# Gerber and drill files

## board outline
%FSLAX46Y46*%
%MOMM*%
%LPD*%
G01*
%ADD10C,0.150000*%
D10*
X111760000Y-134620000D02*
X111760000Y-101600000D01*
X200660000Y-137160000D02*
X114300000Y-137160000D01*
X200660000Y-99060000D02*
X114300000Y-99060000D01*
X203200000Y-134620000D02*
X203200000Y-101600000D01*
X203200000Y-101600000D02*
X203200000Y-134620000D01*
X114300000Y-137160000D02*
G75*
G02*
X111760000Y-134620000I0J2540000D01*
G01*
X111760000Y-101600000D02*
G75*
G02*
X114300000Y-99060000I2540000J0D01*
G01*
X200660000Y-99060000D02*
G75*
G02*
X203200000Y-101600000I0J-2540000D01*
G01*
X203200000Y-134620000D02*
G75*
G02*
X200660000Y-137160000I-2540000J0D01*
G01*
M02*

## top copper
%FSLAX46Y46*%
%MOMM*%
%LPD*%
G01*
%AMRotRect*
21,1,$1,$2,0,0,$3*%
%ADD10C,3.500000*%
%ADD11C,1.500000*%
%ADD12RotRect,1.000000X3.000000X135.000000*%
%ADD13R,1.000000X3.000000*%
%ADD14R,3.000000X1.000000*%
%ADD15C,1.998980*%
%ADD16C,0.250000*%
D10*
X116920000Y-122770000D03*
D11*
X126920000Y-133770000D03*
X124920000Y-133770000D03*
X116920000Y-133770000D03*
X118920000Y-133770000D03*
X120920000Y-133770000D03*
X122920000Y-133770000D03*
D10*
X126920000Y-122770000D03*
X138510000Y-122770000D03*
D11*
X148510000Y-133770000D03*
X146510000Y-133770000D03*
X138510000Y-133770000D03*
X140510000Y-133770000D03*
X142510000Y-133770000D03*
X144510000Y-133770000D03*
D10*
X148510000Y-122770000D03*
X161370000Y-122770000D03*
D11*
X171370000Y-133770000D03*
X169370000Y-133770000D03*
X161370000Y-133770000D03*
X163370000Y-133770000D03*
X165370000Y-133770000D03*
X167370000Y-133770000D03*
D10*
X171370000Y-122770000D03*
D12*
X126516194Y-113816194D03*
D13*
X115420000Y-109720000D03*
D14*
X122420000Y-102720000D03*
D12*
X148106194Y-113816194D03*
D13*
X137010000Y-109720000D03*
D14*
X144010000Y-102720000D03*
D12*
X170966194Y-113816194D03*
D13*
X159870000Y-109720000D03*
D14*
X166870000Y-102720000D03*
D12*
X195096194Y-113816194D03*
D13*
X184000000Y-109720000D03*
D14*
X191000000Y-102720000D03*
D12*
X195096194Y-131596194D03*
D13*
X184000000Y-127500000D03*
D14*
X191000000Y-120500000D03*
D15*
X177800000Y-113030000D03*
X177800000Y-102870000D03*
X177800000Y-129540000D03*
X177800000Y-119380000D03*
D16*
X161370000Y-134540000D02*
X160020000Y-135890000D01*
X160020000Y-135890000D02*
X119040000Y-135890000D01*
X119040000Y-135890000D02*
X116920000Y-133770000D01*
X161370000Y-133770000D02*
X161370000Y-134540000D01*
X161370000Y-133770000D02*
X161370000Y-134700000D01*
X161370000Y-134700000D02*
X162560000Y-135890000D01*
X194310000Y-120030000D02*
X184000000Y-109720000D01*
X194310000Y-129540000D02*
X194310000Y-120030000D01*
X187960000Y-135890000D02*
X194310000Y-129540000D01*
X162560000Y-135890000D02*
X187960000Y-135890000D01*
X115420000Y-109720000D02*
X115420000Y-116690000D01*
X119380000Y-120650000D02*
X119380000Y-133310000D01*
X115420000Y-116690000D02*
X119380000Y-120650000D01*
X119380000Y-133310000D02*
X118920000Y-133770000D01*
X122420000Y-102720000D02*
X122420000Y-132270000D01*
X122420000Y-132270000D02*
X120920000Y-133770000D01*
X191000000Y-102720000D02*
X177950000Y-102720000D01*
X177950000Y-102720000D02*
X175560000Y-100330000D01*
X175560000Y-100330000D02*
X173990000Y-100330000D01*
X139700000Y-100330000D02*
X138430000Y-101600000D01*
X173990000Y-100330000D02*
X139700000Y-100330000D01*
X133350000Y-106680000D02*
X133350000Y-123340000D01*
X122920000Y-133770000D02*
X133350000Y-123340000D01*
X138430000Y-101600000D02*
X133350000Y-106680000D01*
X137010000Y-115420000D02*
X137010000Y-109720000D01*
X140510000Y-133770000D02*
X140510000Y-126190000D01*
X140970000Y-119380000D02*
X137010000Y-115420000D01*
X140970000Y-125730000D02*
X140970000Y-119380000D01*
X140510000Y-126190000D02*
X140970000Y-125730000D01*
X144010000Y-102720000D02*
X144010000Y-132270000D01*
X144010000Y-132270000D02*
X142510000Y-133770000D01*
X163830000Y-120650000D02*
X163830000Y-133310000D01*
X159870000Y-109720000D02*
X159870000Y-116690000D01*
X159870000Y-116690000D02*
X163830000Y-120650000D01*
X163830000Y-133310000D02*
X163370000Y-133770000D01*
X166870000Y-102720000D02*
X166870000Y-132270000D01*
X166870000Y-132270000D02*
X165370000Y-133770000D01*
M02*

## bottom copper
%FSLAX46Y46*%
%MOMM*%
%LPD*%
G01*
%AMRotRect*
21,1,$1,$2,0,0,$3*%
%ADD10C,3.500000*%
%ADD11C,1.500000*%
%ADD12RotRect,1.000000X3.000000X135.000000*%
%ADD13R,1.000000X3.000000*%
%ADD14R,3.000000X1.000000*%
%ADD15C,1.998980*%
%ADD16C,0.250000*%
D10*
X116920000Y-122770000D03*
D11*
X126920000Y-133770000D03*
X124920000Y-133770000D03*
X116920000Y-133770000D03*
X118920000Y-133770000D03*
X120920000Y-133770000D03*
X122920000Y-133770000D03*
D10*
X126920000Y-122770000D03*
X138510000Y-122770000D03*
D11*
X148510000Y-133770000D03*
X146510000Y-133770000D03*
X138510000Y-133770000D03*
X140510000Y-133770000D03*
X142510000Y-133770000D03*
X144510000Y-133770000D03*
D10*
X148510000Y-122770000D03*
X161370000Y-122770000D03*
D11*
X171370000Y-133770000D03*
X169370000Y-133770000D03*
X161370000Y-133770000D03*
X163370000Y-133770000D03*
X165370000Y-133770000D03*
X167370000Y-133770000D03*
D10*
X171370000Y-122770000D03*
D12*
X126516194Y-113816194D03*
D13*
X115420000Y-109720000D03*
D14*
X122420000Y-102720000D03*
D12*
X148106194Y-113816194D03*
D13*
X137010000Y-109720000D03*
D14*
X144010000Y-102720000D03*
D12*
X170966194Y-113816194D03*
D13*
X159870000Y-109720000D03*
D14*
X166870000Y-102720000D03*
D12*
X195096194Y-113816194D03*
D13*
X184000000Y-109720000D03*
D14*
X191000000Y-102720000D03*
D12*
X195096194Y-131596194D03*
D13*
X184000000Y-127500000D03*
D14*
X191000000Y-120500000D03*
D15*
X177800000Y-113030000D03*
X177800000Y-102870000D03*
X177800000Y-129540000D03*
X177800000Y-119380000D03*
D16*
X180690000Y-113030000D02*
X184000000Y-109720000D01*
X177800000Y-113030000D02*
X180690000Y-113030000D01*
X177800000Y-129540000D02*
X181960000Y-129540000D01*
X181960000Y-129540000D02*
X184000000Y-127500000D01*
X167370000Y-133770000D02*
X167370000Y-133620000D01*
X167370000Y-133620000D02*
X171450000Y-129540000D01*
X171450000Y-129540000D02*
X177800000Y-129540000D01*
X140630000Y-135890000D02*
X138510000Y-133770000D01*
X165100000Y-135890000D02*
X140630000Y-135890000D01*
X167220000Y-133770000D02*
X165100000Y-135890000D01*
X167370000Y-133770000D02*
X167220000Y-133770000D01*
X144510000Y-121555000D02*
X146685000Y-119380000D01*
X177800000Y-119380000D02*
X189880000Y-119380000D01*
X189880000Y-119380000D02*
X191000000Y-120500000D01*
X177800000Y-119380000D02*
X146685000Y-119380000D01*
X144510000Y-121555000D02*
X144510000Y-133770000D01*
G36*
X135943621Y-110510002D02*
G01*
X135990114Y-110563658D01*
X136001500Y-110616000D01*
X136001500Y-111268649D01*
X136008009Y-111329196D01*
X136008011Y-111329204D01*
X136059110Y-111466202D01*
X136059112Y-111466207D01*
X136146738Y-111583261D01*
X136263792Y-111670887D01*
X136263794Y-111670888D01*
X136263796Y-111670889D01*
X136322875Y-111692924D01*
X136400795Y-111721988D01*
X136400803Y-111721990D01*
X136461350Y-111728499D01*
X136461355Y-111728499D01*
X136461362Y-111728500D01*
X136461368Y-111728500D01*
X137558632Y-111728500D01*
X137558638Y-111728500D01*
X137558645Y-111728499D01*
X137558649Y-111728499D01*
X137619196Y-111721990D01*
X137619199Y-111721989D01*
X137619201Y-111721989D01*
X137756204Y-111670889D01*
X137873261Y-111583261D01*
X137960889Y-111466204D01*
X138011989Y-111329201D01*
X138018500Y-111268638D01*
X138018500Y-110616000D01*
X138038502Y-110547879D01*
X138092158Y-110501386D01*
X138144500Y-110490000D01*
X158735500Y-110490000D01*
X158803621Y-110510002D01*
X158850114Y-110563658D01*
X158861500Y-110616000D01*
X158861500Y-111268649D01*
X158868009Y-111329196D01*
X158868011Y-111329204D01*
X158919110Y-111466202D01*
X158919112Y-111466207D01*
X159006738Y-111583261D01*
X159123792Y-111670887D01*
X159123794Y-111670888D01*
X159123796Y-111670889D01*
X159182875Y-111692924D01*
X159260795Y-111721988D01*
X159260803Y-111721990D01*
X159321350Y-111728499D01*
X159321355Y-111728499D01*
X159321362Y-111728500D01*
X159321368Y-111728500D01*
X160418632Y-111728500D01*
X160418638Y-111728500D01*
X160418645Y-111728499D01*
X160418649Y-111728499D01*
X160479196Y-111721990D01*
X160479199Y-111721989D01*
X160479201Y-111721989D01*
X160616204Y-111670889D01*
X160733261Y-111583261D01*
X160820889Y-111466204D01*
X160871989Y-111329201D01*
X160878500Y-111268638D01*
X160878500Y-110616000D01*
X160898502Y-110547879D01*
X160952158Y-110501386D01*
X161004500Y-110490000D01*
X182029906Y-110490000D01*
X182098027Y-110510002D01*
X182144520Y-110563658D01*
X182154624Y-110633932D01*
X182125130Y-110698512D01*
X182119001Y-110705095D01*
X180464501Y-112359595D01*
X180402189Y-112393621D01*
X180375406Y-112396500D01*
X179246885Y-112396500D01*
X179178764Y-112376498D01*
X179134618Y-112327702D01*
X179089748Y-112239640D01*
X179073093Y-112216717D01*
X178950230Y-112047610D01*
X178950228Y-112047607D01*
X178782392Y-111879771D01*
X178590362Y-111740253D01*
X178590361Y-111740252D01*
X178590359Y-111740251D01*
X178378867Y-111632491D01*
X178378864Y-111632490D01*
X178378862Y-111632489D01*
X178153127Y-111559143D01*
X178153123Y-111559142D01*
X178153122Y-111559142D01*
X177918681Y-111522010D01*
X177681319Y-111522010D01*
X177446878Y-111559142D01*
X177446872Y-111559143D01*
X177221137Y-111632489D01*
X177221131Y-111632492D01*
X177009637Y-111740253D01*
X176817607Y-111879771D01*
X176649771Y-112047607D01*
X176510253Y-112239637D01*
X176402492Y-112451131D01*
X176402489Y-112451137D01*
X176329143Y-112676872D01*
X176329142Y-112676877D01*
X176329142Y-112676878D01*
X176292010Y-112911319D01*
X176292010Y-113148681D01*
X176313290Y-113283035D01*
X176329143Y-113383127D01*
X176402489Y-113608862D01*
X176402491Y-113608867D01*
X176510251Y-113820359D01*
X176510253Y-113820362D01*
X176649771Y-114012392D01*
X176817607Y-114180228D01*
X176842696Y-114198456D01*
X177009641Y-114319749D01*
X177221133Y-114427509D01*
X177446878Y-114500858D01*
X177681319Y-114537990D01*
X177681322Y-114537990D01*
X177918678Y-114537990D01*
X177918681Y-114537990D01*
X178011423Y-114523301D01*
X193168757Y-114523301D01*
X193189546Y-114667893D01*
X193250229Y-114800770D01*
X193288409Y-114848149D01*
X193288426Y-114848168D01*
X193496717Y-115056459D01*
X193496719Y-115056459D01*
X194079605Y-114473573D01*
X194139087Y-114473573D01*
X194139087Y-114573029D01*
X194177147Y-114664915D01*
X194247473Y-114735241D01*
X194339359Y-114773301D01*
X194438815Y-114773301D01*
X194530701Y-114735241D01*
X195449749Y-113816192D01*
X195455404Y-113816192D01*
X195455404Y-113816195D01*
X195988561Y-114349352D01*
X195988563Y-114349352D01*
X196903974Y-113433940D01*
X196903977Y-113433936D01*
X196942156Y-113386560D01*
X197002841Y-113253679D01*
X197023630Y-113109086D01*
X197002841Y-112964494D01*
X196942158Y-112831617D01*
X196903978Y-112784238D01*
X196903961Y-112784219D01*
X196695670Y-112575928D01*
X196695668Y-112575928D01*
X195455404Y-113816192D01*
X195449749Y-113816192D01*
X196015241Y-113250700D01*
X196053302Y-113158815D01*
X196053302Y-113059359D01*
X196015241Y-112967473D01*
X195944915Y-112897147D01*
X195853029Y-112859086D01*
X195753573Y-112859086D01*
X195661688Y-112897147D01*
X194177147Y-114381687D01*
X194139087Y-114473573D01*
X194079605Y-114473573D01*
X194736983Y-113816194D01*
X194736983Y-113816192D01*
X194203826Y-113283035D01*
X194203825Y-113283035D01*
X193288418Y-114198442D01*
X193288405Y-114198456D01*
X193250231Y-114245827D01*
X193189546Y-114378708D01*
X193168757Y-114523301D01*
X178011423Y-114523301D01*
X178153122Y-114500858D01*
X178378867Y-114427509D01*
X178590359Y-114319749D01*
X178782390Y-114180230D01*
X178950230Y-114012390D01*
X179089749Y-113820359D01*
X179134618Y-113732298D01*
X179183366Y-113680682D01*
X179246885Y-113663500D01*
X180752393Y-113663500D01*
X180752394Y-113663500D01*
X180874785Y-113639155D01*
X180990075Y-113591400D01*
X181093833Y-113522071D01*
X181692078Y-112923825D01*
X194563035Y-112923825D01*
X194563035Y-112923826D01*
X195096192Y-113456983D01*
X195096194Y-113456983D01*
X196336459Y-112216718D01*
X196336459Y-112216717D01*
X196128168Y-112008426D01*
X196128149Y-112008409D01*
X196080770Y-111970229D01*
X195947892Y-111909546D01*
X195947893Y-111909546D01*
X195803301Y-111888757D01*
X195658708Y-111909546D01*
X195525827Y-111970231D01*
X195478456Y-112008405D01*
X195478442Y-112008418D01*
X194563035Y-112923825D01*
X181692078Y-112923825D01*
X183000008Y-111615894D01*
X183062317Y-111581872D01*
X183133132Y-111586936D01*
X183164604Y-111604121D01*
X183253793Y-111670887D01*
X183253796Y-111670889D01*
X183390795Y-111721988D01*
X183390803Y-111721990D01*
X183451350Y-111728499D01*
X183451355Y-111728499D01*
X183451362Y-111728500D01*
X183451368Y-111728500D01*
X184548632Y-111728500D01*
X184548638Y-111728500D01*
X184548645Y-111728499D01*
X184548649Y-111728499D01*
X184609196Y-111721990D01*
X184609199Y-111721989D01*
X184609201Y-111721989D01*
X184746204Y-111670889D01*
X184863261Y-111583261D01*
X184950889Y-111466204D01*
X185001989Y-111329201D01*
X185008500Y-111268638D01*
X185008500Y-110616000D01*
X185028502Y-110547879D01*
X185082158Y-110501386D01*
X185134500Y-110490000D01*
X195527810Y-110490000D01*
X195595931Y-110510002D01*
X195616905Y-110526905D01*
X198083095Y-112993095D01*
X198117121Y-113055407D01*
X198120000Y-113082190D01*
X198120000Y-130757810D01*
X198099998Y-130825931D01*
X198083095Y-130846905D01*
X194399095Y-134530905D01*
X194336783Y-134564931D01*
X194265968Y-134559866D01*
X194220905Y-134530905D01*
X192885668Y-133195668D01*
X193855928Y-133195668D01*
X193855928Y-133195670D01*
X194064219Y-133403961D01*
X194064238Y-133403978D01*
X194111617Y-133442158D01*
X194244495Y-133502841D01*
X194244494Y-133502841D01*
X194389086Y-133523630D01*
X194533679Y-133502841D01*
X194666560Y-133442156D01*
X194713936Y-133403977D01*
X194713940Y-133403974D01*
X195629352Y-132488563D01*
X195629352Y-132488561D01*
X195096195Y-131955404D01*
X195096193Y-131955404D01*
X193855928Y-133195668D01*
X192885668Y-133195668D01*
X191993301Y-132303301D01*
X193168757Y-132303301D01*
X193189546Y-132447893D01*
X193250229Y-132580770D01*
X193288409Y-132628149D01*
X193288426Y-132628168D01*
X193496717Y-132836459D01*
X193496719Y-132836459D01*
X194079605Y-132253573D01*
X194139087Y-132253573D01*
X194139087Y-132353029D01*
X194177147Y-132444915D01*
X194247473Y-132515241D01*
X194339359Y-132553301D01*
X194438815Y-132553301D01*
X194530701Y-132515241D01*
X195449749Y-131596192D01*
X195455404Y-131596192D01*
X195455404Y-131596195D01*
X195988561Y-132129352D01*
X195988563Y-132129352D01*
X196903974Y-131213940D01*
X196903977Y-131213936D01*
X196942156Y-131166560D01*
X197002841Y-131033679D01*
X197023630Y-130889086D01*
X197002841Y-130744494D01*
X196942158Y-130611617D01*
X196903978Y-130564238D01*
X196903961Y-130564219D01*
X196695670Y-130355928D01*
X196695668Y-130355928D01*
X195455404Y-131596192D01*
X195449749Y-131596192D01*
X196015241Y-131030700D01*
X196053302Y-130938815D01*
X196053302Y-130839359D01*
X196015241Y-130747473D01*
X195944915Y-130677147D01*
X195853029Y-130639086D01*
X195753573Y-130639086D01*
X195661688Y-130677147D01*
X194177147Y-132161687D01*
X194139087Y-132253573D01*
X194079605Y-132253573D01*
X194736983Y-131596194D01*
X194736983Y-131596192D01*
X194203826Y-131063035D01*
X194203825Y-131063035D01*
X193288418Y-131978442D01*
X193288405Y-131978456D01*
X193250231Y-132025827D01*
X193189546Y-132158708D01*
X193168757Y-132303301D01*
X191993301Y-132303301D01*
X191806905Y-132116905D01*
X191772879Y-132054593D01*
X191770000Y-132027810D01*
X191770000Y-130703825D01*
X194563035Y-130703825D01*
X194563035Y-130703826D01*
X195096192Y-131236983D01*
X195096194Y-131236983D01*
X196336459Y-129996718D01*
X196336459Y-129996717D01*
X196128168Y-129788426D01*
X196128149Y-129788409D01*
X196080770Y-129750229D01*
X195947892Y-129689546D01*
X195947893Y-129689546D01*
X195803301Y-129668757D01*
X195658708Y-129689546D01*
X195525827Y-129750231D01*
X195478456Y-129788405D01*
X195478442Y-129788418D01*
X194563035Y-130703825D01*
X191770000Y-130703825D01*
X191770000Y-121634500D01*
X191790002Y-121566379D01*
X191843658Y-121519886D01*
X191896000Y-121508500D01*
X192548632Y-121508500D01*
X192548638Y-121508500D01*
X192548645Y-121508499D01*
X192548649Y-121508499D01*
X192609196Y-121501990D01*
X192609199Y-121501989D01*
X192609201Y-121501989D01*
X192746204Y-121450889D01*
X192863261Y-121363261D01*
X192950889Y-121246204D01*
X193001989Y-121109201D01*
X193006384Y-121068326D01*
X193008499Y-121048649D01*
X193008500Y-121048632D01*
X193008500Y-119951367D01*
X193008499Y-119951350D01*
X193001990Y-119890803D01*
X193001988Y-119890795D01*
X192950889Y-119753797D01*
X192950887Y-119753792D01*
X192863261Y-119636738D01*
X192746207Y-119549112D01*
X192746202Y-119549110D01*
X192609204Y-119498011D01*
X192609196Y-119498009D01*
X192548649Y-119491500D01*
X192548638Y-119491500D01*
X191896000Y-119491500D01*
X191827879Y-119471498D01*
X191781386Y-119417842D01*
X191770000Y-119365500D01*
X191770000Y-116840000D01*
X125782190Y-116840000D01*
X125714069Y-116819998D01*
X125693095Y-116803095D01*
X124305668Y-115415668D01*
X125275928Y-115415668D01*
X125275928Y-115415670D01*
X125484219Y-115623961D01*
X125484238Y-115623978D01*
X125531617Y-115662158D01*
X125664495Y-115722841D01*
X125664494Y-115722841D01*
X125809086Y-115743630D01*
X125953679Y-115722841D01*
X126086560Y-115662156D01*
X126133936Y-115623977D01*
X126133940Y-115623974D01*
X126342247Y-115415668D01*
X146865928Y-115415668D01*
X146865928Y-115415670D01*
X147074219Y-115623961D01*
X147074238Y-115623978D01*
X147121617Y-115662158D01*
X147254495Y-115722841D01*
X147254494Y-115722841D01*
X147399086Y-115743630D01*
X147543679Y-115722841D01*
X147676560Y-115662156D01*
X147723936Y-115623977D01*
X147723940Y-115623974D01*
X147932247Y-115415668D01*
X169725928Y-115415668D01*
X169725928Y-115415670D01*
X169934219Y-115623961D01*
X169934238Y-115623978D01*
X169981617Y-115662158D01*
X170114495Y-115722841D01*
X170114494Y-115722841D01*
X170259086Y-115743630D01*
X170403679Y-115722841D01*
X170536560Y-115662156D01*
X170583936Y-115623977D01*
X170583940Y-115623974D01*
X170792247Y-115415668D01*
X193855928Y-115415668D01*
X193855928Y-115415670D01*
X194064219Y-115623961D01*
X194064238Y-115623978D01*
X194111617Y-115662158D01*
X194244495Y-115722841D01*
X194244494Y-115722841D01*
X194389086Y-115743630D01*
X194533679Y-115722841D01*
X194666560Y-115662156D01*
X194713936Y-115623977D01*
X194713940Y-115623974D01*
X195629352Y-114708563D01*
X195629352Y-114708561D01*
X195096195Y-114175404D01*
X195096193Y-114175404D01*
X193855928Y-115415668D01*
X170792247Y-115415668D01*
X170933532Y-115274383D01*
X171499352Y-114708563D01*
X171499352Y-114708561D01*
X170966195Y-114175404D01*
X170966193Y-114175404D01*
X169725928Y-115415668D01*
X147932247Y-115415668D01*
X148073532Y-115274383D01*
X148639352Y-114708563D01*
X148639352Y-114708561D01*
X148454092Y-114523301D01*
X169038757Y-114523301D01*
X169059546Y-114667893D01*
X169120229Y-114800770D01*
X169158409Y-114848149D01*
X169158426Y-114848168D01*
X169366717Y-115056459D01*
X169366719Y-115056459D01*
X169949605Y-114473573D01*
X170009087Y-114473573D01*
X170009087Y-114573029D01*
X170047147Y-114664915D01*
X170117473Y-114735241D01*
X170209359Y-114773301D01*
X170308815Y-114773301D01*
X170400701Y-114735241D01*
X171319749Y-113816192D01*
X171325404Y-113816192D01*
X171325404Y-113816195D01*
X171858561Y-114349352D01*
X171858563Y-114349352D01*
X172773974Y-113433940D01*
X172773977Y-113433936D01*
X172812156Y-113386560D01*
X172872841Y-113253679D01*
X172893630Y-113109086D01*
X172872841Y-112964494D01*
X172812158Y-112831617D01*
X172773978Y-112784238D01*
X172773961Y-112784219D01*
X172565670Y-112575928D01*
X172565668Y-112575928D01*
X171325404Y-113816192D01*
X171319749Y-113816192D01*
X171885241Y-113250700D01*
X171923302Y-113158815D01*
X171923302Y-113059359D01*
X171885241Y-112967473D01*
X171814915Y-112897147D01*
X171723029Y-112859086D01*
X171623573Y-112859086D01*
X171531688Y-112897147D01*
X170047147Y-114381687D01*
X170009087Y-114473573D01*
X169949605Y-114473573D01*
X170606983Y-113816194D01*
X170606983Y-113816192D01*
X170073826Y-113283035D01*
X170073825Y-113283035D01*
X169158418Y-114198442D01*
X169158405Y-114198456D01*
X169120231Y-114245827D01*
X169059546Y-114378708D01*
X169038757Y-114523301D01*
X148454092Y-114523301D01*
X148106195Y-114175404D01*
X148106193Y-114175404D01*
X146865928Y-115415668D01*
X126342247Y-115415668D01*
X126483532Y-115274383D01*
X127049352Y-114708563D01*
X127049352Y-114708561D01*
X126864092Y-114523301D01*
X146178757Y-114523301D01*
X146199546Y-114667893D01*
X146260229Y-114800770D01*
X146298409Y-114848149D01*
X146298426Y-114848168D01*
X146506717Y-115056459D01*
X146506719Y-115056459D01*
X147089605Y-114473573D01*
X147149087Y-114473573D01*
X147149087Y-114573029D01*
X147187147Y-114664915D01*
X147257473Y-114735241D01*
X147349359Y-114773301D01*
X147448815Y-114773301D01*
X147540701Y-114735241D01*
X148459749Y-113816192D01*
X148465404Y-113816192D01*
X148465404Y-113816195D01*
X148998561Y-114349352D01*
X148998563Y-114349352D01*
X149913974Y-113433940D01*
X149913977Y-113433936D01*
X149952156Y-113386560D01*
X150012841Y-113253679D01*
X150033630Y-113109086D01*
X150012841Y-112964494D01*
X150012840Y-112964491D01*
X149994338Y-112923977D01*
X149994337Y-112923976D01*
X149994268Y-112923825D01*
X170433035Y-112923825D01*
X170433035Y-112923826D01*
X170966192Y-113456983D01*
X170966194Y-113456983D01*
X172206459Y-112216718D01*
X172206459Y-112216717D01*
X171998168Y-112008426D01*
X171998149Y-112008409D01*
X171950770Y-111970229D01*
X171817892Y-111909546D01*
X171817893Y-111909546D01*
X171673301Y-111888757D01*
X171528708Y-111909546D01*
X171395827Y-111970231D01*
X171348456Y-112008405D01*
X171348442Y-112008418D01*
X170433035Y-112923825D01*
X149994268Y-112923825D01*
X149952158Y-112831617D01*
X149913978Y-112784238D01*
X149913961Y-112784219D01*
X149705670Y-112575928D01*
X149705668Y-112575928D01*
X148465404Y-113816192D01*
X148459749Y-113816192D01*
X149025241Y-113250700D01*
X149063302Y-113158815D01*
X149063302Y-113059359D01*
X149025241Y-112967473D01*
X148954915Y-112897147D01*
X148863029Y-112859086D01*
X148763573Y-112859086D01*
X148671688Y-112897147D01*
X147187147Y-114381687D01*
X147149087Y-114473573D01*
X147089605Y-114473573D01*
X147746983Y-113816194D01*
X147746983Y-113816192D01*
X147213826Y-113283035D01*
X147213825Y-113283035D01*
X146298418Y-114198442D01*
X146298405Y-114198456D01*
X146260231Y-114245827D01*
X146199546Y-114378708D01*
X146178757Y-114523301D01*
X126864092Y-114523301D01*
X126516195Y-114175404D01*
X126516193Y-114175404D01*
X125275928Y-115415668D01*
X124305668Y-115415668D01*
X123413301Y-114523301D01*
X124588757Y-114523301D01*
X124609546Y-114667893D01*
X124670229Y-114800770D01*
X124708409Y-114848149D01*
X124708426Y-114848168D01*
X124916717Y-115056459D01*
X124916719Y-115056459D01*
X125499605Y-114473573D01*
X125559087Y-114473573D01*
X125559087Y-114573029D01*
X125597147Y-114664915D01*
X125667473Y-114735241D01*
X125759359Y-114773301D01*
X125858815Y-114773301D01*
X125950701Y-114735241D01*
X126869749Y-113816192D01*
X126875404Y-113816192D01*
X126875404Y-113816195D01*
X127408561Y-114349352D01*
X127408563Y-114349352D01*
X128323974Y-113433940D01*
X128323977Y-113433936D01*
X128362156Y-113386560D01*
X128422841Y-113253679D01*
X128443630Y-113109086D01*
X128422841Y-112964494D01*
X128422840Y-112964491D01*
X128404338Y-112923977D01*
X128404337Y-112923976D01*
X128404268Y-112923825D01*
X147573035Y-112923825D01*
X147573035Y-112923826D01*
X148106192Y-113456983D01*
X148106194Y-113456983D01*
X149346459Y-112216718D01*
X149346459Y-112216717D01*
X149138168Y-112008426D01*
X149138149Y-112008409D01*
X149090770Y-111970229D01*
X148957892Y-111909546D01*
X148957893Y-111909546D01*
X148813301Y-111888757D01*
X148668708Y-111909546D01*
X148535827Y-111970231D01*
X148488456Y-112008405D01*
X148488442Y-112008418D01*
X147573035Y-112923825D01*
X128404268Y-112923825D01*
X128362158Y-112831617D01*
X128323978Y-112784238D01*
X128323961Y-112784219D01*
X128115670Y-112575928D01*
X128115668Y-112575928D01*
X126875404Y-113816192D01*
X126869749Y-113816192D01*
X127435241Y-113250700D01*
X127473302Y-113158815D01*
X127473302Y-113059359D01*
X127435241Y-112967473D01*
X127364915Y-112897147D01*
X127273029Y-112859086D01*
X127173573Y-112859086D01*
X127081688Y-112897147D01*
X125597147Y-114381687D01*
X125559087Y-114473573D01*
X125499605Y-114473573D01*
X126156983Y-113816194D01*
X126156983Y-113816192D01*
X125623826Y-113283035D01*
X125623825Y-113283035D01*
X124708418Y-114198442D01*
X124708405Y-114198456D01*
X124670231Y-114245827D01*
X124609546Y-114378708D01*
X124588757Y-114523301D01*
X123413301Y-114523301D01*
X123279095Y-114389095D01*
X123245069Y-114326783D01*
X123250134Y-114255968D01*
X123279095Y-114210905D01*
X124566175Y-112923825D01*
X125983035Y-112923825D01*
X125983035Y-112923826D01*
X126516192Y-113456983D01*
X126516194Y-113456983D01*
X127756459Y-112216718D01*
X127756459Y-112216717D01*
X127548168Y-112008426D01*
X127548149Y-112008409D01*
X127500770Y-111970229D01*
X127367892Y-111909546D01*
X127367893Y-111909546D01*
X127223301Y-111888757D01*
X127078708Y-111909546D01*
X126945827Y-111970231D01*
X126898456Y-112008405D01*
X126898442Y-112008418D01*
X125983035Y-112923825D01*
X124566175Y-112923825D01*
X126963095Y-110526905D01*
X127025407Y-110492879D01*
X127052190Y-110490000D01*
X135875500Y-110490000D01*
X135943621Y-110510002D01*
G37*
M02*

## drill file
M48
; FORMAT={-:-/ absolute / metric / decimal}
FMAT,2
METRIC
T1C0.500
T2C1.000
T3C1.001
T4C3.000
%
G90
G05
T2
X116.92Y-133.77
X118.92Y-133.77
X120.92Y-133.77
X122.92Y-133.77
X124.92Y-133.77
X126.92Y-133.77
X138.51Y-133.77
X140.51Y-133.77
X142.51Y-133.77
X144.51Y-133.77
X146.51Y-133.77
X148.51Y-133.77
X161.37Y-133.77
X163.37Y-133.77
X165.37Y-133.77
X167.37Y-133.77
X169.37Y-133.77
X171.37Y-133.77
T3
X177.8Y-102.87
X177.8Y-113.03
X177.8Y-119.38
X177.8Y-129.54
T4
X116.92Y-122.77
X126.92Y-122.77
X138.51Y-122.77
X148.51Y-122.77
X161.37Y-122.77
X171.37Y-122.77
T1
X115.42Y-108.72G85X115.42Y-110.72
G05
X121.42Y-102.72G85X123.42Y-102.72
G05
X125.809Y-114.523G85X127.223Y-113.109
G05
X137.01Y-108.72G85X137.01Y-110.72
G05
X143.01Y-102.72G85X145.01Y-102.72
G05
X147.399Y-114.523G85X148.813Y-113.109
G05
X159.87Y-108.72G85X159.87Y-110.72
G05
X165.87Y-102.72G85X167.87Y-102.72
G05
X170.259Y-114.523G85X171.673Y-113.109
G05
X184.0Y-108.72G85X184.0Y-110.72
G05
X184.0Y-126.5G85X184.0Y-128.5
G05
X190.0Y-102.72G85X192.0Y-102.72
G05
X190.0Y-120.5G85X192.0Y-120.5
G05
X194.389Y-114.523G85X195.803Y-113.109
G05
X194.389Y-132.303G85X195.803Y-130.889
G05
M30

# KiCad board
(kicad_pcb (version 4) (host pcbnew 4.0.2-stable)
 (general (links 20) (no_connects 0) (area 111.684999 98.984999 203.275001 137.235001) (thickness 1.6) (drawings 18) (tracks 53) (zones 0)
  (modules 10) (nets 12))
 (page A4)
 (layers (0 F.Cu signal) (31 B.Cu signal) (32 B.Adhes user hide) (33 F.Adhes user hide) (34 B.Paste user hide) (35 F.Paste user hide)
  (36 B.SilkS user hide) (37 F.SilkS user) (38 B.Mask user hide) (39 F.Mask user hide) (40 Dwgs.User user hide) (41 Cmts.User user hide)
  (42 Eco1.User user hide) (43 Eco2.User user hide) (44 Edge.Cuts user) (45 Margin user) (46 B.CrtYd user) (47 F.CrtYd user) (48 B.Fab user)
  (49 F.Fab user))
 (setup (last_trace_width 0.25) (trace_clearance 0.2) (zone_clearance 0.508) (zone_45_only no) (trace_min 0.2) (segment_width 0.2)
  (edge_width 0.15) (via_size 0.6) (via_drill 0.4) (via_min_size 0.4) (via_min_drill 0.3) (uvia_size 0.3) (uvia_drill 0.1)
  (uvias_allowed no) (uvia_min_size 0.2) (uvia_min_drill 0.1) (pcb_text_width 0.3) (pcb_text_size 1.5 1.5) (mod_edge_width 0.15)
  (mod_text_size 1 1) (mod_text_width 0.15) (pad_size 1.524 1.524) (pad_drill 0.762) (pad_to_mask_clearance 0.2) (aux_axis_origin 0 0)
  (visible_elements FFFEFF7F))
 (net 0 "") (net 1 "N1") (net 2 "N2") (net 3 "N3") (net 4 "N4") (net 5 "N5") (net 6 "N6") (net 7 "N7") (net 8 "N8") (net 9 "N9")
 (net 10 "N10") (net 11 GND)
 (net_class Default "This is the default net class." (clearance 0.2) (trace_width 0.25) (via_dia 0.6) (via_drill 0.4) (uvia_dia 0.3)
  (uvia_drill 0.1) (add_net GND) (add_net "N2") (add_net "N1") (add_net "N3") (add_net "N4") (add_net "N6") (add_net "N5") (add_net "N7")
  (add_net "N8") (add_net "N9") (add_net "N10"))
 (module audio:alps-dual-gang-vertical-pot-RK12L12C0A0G (layer F.Cu) (at 121.92 128.27)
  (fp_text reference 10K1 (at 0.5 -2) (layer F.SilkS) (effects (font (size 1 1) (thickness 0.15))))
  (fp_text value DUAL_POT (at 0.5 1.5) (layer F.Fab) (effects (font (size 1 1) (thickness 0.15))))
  (pad b thru_hole circle (at -5 -5.5) (size 3.5 3.5) (drill 3) (layers *.Cu *.Mask F.SilkS))
  (pad 3 thru_hole circle (at 5 5.5) (size 1.5 1.5) (drill 1) (layers *.Cu *.Mask F.SilkS))
  (pad 6 thru_hole circle (at 3 5.5) (size 1.5 1.5) (drill 1) (layers *.Cu *.Mask F.SilkS))
  (pad 2 thru_hole circle (at -5 5.5) (size 1.5 1.5) (drill 1) (layers *.Cu *.Mask F.SilkS) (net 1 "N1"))
  (pad 1 thru_hole circle (at -3 5.5) (size 1.5 1.5) (drill 1) (layers *.Cu *.Mask F.SilkS) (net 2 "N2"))
  (pad 4 thru_hole circle (at -1 5.5) (size 1.5 1.5) (drill 1) (layers *.Cu *.Mask F.SilkS) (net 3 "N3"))
  (pad 5 thru_hole circle (at 1 5.5) (size 1.5 1.5) (drill 1) (layers *.Cu *.Mask F.SilkS) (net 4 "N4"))
  (pad a thru_hole circle (at 5 -5.5) (size 3.5 3.5) (drill 3) (layers *.Cu *.Mask F.SilkS)))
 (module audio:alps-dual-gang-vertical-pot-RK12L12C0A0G (layer F.Cu) (at 143.51 128.27)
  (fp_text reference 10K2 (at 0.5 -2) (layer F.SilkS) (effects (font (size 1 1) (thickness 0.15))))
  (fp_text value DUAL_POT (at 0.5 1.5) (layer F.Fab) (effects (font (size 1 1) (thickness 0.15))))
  (pad b thru_hole circle (at -5 -5.5) (size 3.5 3.5) (drill 3) (layers *.Cu *.Mask F.SilkS))
  (pad 3 thru_hole circle (at 5 5.5) (size 1.5 1.5) (drill 1) (layers *.Cu *.Mask F.SilkS))
  (pad 6 thru_hole circle (at 3 5.5) (size 1.5 1.5) (drill 1) (layers *.Cu *.Mask F.SilkS))
  (pad 2 thru_hole circle (at -5 5.5) (size 1.5 1.5) (drill 1) (layers *.Cu *.Mask F.SilkS) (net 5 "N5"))
  (pad 1 thru_hole circle (at -3 5.5) (size 1.5 1.5) (drill 1) (layers *.Cu *.Mask F.SilkS) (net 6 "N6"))
  (pad 4 thru_hole circle (at -1 5.5) (size 1.5 1.5) (drill 1) (layers *.Cu *.Mask F.SilkS) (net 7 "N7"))
  (pad 5 thru_hole circle (at 1 5.5) (size 1.5 1.5) (drill 1) (layers *.Cu *.Mask F.SilkS) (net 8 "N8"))
  (pad a thru_hole circle (at 5 -5.5) (size 3.5 3.5) (drill 3) (layers *.Cu *.Mask F.SilkS)))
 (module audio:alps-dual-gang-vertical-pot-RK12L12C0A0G (layer F.Cu) (at 166.37 128.27)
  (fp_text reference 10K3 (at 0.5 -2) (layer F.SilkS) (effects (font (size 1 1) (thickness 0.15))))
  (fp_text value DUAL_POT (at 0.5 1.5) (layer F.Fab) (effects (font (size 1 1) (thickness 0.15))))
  (pad b thru_hole circle (at -5 -5.5) (size 3.5 3.5) (drill 3) (layers *.Cu *.Mask F.SilkS))
  (pad 3 thru_hole circle (at 5 5.5) (size 1.5 1.5) (drill 1) (layers *.Cu *.Mask F.SilkS))
  (pad 6 thru_hole circle (at 3 5.5) (size 1.5 1.5) (drill 1) (layers *.Cu *.Mask F.SilkS))
  (pad 2 thru_hole circle (at -5 5.5) (size 1.5 1.5) (drill 1) (layers *.Cu *.Mask F.SilkS) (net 1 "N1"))
  (pad 1 thru_hole circle (at -3 5.5) (size 1.5 1.5) (drill 1) (layers *.Cu *.Mask F.SilkS) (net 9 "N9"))
  (pad 4 thru_hole circle (at -1 5.5) (size 1.5 1.5) (drill 1) (layers *.Cu *.Mask F.SilkS) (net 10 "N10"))
  (pad 5 thru_hole circle (at 1 5.5) (size 1.5 1.5) (drill 1) (layers *.Cu *.Mask F.SilkS) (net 5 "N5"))
  (pad a thru_hole circle (at 5 -5.5) (size 3.5 3.5) (drill 3) (layers *.Cu *.Mask F.SilkS)))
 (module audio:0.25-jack (layer F.Cu) (at 121.92 109.22)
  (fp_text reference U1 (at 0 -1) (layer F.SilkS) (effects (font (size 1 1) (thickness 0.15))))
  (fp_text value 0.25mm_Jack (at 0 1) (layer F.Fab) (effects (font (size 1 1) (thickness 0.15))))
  (pad 3 thru_hole rect (at 4.596194 4.596194 135) (size 1 3) (drill oval 0.5 2.5) (layers *.Cu *.Mask F.SilkS) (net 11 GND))
  (pad 1 thru_hole rect (at -6.5 0.5) (size 1 3) (drill oval 0.5 2.5) (layers *.Cu *.Mask F.SilkS) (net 2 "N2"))
  (pad 2 thru_hole rect (at 0.5 -6.5 90) (size 1 3) (drill oval 0.5 2.5) (layers *.Cu *.Mask F.SilkS) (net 3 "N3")))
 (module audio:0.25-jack (layer F.Cu) (at 143.51 109.22)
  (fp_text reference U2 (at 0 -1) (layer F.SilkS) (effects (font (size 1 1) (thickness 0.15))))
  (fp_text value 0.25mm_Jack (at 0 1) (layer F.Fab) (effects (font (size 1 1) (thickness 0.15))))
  (pad 3 thru_hole rect (at 4.596194 4.596194 135) (size 1 3) (drill oval 0.5 2.5) (layers *.Cu *.Mask F.SilkS) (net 11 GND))
  (pad 1 thru_hole rect (at -6.5 0.5) (size 1 3) (drill oval 0.5 2.5) (layers *.Cu *.Mask F.SilkS) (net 6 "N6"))
  (pad 2 thru_hole rect (at 0.5 -6.5 90) (size 1 3) (drill oval 0.5 2.5) (layers *.Cu *.Mask F.SilkS) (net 7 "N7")))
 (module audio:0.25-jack (layer F.Cu) (at 166.37 109.22)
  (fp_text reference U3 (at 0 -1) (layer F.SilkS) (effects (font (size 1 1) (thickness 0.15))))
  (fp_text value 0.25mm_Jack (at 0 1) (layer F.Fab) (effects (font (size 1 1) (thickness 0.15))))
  (pad 3 thru_hole rect (at 4.596194 4.596194 135) (size 1 3) (drill oval 0.5 2.5) (layers *.Cu *.Mask F.SilkS) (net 11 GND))
  (pad 1 thru_hole rect (at -6.5 0.5) (size 1 3) (drill oval 0.5 2.5) (layers *.Cu *.Mask F.SilkS) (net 9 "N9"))
  (pad 2 thru_hole rect (at 0.5 -6.5 90) (size 1 3) (drill oval 0.5 2.5) (layers *.Cu *.Mask F.SilkS) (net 10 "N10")))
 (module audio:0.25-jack (layer F.Cu) (at 190.5 109.22)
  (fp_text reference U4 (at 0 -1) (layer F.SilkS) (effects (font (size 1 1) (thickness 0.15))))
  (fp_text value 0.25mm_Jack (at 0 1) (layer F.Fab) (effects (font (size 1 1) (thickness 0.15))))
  (pad 3 thru_hole rect (at 4.596194 4.596194 135) (size 1 3) (drill oval 0.5 2.5) (layers *.Cu *.Mask F.SilkS) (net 11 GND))
  (pad 1 thru_hole rect (at -6.5 0.5) (size 1 3) (drill oval 0.5 2.5) (layers *.Cu *.Mask F.SilkS) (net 1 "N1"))
  (pad 2 thru_hole rect (at 0.5 -6.5 90) (size 1 3) (drill oval 0.5 2.5) (layers *.Cu *.Mask F.SilkS) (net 4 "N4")))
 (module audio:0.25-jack (layer F.Cu) (at 190.5 127)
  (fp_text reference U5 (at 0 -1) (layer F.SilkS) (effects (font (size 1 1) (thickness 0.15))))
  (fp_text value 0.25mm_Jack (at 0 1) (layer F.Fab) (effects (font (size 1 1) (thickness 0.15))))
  (pad 3 thru_hole rect (at 4.596194 4.596194 135) (size 1 3) (drill oval 0.5 2.5) (layers *.Cu *.Mask F.SilkS) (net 11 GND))
  (pad 1 thru_hole rect (at -6.5 0.5) (size 1 3) (drill oval 0.5 2.5) (layers *.Cu *.Mask F.SilkS) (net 5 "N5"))
  (pad 2 thru_hole rect (at 0.5 -6.5 90) (size 1 3) (drill oval 0.5 2.5) (layers *.Cu *.Mask F.SilkS) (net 8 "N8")))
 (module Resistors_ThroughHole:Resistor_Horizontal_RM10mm (layer F.Cu) (at 177.8 113.03 90)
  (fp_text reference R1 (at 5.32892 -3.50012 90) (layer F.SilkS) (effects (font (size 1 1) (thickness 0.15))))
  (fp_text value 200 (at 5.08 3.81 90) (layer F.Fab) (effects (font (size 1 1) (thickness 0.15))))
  (pad 1 thru_hole circle (at 0 0 90) (size 1.99898 1.99898) (drill 1.00076) (layers *.Cu *.SilkS *.Mask) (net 1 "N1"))
  (pad 2 thru_hole circle (at 10.16 0 90) (size 1.99898 1.99898) (drill 1.00076) (layers *.Cu *.SilkS *.Mask) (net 4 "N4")))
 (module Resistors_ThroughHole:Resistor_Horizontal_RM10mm (layer F.Cu) (at 177.8 129.54 90)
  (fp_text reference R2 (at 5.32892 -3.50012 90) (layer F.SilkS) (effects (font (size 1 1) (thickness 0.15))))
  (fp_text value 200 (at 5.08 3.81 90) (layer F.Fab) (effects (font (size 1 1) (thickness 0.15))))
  (pad 1 thru_hole circle (at 0 0 90) (size 1.99898 1.99898) (drill 1.00076) (layers *.Cu *.SilkS *.Mask) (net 5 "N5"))
  (pad 2 thru_hole circle (at 10.16 0 90) (size 1.99898 1.99898) (drill 1.00076) (layers *.Cu *.SilkS *.Mask) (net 8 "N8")))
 (gr_line (start 111.76 134.62) (end 111.76 101.6) (angle 90) (layer Edge.Cuts) (width 0.15))
 (gr_line (start 200.66 137.16) (end 114.3 137.16) (angle 90) (layer Edge.Cuts) (width 0.15))
 (gr_line (start 200.66 99.06) (end 114.3 99.06) (angle 90) (layer Edge.Cuts) (width 0.15))
 (gr_line (start 203.2 134.62) (end 203.2 101.6) (angle 90) (layer Edge.Cuts) (width 0.15))
 (gr_line (start 203.2 101.6) (end 203.2 134.62) (angle 90) (layer Edge.Cuts) (width 0.15))
 (gr_arc (start 114.3 134.62) (end 114.3 137.16) (angle 90) (layer Edge.Cuts) (width 0.15))
 (gr_arc (start 114.3 101.6) (end 111.76 101.6) (angle 90) (layer Edge.Cuts) (width 0.15))
 (gr_arc (start 200.66 101.6) (end 200.66 99.06) (angle 90) (layer Edge.Cuts) (width 0.15))
 (gr_arc (start 200.66 134.62) (end 203.2 134.62) (angle 90) (layer Edge.Cuts) (width 0.15))
 (segment (start 161.37 134.54) (end 160.02 135.89) (width 0.25) (layer F.Cu) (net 1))
 (segment (start 160.02 135.89) (end 119.04 135.89) (width 0.25) (layer F.Cu) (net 1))
 (segment (start 119.04 135.89) (end 116.92 133.77) (width 0.25) (layer F.Cu) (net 1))
 (segment (start 161.37 133.77) (end 161.37 134.54) (width 0.25) (layer F.Cu) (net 1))
 (segment (start 161.37 133.77) (end 161.37 134.7) (width 0.25) (layer F.Cu) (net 1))
 (segment (start 161.37 134.7) (end 162.56 135.89) (width 0.25) (layer F.Cu) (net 1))
 (segment (start 194.31 120.03) (end 184 109.72) (width 0.25) (layer F.Cu) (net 1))
 (segment (start 180.69 113.03) (end 184 109.72) (width 0.25) (layer B.Cu) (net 1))
 (segment (start 177.8 113.03) (end 180.69 113.03) (width 0.25) (layer B.Cu) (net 1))
 (segment (start 194.31 129.54) (end 194.31 120.03) (width 0.25) (layer F.Cu) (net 1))
 (segment (start 187.96 135.89) (end 194.31 129.54) (width 0.25) (layer F.Cu) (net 1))
 (segment (start 162.56 135.89) (end 187.96 135.89) (width 0.25) (layer F.Cu) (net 1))
 (segment (start 115.42 109.72) (end 115.42 116.69) (width 0.25) (layer F.Cu) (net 2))
 (segment (start 119.38 120.65) (end 119.38 133.31) (width 0.25) (layer F.Cu) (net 2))
 (segment (start 115.42 116.69) (end 119.38 120.65) (width 0.25) (layer F.Cu) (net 2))
 (segment (start 119.38 133.31) (end 118.92 133.77) (width 0.25) (layer F.Cu) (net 2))
 (segment (start 122.42 102.72) (end 122.42 132.27) (width 0.25) (layer F.Cu) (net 3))
 (segment (start 122.42 132.27) (end 120.92 133.77) (width 0.25) (layer F.Cu) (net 3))
 (segment (start 191 102.72) (end 177.95 102.72) (width 0.25) (layer F.Cu) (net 4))
 (segment (start 177.95 102.72) (end 175.56 100.33) (width 0.25) (layer F.Cu) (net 4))
 (segment (start 175.56 100.33) (end 173.99 100.33) (width 0.25) (layer F.Cu) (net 4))
 (segment (start 139.7 100.33) (end 138.43 101.6) (width 0.25) (layer F.Cu) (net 4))
 (segment (start 173.99 100.33) (end 139.7 100.33) (width 0.25) (layer F.Cu) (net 4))
 (segment (start 133.35 106.68) (end 133.35 123.34) (width 0.25) (layer F.Cu) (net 4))
 (segment (start 122.92 133.77) (end 133.35 123.34) (width 0.25) (layer F.Cu) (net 4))
 (segment (start 138.43 101.6) (end 133.35 106.68) (width 0.25) (layer F.Cu) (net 4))
 (segment (start 177.8 129.54) (end 181.96 129.54) (width 0.25) (layer B.Cu) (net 5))
 (segment (start 181.96 129.54) (end 184 127.5) (width 0.25) (layer B.Cu) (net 5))
 (segment (start 167.37 133.77) (end 167.37 133.62) (width 0.25) (layer B.Cu) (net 5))
 (segment (start 167.37 133.62) (end 171.45 129.54) (width 0.25) (layer B.Cu) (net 5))
 (segment (start 171.45 129.54) (end 177.8 129.54) (width 0.25) (layer B.Cu) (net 5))
 (segment (start 140.63 135.89) (end 138.51 133.77) (width 0.25) (layer B.Cu) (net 5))
 (segment (start 165.1 135.89) (end 140.63 135.89) (width 0.25) (layer B.Cu) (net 5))
 (segment (start 167.22 133.77) (end 165.1 135.89) (width 0.25) (layer B.Cu) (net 5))
 (segment (start 167.37 133.77) (end 167.22 133.77) (width 0.25) (layer B.Cu) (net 5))
 (segment (start 137.01 115.42) (end 137.01 109.72) (width 0.25) (layer F.Cu) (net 6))
 (segment (start 140.51 133.77) (end 140.51 126.19) (width 0.25) (layer F.Cu) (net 6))
 (segment (start 140.97 119.38) (end 137.01 115.42) (width 0.25) (layer F.Cu) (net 6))
 (segment (start 140.97 125.73) (end 140.97 119.38) (width 0.25) (layer F.Cu) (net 6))
 (segment (start 140.51 126.19) (end 140.97 125.73) (width 0.25) (layer F.Cu) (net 6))
 (segment (start 144.01 102.72) (end 144.01 132.27) (width 0.25) (layer F.Cu) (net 7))
 (segment (start 144.01 132.27) (end 142.51 133.77) (width 0.25) (layer F.Cu) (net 7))
 (segment (start 144.51 121.555) (end 146.685 119.38) (width 0.25) (layer B.Cu) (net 8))
 (segment (start 177.8 119.38) (end 189.88 119.38) (width 0.25) (layer B.Cu) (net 8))
 (segment (start 189.88 119.38) (end 191 120.5) (width 0.25) (layer B.Cu) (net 8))
 (segment (start 177.8 119.38) (end 146.685 119.38) (width 0.25) (layer B.Cu) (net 8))
 (segment (start 144.51 121.555) (end 144.51 133.77) (width 0.25) (layer B.Cu) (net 8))
 (segment (start 163.83 120.65) (end 163.83 133.31) (width 0.25) (layer F.Cu) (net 9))
 (segment (start 159.87 109.72) (end 159.87 116.69) (width 0.25) (layer F.Cu) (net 9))
 (segment (start 159.87 116.69) (end 163.83 120.65) (width 0.25) (layer F.Cu) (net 9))
 (segment (start 163.83 133.31) (end 163.37 133.77) (width 0.25) (layer F.Cu) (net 9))
 (segment (start 166.87 102.72) (end 166.87 132.27) (width 0.25) (layer F.Cu) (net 10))
 (segment (start 166.87 132.27) (end 165.37 133.77) (width 0.25) (layer F.Cu) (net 10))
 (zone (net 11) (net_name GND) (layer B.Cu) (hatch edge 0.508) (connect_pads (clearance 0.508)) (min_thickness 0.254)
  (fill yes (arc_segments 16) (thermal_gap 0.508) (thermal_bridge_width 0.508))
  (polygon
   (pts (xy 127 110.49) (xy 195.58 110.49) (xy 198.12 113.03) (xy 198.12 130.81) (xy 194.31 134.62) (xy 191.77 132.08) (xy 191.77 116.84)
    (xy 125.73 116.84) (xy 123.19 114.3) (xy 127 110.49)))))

